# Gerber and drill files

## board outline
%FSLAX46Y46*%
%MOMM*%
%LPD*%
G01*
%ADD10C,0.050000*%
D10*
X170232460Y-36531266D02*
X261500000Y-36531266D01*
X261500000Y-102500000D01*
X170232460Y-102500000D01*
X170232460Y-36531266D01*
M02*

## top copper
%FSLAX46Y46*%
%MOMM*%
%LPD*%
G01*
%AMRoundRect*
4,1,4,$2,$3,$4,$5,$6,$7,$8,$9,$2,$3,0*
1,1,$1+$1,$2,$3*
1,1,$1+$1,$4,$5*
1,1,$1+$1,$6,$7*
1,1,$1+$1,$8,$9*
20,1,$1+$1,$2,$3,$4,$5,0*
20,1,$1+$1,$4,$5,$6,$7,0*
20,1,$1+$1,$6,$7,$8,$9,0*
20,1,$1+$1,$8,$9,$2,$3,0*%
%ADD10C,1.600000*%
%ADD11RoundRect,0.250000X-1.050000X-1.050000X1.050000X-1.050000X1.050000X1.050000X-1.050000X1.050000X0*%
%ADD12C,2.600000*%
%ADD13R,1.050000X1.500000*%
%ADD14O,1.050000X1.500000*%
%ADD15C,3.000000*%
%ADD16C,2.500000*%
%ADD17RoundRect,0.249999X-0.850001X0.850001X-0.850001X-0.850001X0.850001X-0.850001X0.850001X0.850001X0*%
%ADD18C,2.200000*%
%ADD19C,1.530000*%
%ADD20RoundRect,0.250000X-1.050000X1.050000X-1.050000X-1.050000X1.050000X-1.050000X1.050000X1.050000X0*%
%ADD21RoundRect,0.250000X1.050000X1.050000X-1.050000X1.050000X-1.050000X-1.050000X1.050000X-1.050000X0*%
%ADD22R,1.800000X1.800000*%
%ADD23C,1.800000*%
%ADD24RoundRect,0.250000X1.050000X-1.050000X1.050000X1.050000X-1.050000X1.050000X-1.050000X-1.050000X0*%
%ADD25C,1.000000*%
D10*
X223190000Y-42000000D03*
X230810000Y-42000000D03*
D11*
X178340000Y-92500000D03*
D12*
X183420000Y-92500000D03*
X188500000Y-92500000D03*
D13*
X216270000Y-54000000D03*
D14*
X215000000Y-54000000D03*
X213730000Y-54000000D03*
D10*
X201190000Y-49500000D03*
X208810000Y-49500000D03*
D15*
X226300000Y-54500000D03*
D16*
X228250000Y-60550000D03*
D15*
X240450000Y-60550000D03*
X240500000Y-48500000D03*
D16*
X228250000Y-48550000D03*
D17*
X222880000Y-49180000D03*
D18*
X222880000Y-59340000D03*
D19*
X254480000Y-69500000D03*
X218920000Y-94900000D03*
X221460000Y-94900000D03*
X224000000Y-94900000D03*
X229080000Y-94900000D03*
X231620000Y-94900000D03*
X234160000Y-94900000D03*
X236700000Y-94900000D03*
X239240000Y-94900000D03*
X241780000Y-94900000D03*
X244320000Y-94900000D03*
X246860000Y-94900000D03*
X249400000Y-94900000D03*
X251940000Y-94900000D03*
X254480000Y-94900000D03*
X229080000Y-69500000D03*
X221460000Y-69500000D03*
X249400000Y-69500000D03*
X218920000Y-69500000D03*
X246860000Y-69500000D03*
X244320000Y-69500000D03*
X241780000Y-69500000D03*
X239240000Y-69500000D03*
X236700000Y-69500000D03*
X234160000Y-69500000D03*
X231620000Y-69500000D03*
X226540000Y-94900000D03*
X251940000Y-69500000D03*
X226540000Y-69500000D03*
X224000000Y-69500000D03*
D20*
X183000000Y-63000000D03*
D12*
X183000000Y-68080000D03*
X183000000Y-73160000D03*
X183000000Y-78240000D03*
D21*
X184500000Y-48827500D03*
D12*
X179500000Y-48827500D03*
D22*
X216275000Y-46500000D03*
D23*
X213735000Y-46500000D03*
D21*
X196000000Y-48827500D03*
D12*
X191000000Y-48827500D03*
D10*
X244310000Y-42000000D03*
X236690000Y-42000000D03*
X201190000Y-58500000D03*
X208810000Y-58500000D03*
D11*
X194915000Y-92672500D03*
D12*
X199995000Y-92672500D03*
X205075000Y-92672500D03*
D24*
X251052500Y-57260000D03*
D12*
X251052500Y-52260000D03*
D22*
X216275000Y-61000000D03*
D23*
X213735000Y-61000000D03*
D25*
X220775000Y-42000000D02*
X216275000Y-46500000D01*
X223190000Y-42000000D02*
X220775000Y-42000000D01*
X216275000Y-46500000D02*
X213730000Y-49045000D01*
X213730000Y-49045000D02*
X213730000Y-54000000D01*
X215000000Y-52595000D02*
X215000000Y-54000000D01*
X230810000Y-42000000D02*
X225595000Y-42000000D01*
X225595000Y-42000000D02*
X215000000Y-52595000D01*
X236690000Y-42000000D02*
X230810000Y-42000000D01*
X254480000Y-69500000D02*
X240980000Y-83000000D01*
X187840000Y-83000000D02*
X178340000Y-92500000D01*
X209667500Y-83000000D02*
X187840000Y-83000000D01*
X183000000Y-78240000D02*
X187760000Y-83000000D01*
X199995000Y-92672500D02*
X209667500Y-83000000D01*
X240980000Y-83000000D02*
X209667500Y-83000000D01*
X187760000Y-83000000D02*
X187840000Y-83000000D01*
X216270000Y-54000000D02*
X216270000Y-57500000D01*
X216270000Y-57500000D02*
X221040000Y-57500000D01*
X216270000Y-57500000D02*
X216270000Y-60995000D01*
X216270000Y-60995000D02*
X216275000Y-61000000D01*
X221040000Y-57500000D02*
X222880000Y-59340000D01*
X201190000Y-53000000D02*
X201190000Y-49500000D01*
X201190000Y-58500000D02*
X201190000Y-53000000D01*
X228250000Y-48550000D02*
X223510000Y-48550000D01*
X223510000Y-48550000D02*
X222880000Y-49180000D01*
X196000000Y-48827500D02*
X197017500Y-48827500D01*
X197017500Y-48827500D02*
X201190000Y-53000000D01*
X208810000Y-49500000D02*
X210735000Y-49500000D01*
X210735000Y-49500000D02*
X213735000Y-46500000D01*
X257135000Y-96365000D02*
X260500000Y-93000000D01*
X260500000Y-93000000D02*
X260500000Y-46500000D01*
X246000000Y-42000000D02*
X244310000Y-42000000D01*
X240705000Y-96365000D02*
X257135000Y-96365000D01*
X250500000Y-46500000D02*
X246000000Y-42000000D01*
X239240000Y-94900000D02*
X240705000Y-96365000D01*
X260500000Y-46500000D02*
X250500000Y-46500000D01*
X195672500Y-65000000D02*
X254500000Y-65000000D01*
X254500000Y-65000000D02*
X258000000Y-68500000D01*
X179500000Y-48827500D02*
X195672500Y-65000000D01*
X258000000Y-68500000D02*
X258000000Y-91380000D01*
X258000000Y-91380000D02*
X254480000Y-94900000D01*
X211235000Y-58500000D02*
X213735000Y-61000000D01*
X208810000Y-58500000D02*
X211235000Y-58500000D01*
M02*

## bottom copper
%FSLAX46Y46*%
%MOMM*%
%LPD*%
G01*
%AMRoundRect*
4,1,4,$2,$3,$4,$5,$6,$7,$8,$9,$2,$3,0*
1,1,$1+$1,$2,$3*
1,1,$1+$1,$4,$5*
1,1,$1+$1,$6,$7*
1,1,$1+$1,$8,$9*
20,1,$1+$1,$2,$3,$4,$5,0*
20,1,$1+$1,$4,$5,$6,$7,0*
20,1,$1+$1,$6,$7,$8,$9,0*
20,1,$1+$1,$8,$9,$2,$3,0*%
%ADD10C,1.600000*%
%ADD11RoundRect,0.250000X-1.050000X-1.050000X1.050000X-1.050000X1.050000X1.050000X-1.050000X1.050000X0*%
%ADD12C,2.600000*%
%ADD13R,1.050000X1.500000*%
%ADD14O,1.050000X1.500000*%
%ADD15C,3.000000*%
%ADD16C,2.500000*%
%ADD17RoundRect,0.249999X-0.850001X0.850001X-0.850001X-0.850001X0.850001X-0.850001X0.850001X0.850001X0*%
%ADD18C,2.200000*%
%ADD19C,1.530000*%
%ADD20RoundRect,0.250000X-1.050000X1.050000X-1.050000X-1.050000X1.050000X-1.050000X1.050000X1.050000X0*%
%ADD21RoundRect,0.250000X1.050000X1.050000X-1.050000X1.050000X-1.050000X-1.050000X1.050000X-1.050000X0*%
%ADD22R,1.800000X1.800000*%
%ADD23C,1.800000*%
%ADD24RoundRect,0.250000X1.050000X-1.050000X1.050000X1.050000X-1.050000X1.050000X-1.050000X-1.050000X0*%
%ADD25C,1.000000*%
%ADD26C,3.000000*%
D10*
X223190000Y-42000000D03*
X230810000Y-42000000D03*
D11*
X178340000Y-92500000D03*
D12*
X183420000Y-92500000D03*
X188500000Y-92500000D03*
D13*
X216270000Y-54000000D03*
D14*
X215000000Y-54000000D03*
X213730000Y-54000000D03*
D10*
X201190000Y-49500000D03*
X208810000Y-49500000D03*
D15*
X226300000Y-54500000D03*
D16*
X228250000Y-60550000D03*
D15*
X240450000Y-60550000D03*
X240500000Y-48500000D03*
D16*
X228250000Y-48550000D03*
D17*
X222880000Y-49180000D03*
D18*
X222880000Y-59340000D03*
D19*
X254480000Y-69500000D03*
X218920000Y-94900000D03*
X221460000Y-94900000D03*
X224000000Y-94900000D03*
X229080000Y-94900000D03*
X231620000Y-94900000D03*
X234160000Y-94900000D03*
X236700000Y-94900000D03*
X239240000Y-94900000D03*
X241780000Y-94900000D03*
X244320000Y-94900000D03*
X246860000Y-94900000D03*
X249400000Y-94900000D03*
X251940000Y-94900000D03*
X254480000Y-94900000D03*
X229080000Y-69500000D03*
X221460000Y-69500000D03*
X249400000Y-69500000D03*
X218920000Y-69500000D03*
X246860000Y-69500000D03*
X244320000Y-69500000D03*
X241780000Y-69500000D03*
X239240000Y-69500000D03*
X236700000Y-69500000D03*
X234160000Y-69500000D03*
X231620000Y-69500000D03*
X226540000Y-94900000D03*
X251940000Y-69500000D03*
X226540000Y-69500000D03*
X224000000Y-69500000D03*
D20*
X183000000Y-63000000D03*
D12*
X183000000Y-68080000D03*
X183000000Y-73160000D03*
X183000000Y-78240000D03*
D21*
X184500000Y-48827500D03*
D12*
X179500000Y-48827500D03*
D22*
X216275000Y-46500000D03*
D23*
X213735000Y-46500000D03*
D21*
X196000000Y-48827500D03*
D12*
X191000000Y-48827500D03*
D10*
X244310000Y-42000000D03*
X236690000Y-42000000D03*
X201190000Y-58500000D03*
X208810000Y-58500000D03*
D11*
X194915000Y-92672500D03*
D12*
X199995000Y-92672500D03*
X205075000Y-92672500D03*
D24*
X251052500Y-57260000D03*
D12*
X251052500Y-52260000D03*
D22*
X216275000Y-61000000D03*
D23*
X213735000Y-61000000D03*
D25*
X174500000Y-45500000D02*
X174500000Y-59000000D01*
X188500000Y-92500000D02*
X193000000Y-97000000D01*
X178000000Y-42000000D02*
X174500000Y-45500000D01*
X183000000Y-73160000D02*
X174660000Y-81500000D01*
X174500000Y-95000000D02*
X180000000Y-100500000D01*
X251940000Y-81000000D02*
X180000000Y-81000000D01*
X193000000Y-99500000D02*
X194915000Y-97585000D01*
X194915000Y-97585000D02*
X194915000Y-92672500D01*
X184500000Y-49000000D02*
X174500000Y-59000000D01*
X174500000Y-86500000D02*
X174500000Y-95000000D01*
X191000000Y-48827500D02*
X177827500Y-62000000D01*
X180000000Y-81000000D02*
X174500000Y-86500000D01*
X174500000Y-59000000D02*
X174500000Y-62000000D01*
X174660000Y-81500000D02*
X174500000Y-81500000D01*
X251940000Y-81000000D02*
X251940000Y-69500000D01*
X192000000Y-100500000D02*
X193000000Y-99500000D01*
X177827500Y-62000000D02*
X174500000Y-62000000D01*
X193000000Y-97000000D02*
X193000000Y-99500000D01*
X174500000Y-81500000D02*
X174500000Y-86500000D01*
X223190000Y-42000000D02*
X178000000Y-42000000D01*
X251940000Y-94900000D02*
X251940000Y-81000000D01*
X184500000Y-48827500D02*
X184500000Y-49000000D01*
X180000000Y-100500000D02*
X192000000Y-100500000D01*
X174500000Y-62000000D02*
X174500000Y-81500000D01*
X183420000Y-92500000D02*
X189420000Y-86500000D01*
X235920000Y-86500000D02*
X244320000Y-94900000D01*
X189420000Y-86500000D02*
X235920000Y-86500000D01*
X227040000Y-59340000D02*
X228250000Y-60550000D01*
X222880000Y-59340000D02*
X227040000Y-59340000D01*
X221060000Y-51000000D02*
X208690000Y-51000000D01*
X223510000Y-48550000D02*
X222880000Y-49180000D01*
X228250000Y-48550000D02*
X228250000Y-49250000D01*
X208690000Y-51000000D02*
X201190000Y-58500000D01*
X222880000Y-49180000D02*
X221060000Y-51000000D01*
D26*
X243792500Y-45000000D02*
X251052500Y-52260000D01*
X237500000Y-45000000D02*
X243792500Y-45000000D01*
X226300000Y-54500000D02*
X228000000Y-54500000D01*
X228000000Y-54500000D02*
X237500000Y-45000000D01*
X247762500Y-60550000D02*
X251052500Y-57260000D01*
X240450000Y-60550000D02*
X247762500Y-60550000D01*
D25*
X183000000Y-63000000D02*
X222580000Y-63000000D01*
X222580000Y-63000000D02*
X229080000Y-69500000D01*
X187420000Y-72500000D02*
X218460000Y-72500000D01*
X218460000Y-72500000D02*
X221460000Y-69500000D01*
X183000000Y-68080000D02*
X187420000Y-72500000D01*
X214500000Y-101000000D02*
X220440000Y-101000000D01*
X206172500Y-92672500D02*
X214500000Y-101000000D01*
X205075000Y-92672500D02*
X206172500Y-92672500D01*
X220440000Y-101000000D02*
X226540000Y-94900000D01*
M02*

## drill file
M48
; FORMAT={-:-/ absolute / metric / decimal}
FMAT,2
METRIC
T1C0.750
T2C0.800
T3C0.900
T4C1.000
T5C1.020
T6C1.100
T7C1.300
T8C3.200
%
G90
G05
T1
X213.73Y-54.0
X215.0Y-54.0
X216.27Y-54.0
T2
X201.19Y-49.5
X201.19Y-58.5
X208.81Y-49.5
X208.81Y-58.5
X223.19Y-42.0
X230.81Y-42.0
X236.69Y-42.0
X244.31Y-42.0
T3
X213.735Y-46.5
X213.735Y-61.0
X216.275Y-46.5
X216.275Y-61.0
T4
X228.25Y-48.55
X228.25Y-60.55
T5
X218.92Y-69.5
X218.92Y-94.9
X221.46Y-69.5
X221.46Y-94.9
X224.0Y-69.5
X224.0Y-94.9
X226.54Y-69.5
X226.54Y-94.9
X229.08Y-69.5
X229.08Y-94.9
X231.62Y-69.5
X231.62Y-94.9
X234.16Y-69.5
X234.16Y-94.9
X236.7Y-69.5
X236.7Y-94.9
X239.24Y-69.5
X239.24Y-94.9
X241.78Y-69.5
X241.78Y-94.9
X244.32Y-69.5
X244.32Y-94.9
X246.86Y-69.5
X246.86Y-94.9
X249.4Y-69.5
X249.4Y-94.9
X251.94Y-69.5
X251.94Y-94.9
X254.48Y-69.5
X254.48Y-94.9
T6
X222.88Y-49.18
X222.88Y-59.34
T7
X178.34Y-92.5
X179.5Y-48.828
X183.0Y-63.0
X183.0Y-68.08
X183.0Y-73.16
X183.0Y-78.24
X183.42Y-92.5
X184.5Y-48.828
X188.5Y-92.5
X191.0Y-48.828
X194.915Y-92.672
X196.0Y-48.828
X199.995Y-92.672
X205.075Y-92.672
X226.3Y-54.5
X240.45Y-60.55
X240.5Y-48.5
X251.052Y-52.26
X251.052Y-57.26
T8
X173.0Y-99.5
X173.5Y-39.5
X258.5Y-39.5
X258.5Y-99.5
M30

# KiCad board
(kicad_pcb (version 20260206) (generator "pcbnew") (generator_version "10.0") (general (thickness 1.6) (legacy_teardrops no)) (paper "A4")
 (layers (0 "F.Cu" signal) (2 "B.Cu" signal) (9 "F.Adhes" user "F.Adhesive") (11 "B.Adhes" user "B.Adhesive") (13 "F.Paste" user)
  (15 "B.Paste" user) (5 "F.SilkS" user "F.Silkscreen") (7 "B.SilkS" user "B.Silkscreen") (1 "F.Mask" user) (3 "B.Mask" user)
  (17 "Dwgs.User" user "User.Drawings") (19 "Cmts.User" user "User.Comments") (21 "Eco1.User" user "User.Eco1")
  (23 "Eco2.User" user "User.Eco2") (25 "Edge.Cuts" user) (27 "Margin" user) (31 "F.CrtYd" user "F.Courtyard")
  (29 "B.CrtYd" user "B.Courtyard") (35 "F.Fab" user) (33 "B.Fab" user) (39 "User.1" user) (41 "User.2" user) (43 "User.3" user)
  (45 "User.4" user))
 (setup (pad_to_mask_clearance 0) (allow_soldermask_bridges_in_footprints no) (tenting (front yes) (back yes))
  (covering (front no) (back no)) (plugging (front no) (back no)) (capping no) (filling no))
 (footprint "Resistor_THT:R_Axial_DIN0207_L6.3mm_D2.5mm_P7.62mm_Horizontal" (layer "F.Cu") (at 223.19 42)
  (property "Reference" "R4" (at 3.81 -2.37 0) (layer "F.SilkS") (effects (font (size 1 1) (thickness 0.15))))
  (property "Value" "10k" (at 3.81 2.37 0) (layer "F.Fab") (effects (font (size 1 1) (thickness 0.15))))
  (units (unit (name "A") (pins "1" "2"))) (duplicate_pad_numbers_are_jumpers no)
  (pad "1" thru_hole circle (at 0 0) (size 1.6 1.6) (drill 0.8) (layers "*.Cu" "*.Mask") (remove_unused_layers no) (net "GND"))
  (pad "2" thru_hole circle (at 7.62 0) (size 1.6 1.6) (drill 0.8) (layers "*.Cu" "*.Mask") (remove_unused_layers no) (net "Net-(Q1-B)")))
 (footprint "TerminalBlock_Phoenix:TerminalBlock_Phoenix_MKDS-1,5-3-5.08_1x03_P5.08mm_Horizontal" (layer "F.Cu") (at 178.34 92.5)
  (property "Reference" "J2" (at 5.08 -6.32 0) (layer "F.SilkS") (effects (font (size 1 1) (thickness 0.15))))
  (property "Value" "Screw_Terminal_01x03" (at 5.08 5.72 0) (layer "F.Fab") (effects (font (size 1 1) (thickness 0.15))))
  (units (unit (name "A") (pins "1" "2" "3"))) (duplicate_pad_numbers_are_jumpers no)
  (pad "1" thru_hole roundrect (at 0 0) (size 2.6 2.6) (drill 1.3) (layers "*.Cu" "*.Mask") (remove_unused_layers no)
   (roundrect_rratio 0.096154) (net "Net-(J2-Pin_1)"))
  (pad "2" thru_hole circle (at 5.08 0) (size 2.6 2.6) (drill 1.3) (layers "*.Cu" "*.Mask") (remove_unused_layers no) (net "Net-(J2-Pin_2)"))
  (pad "3" thru_hole circle (at 10.16 0) (size 2.6 2.6) (drill 1.3) (layers "*.Cu" "*.Mask") (remove_unused_layers no) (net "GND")))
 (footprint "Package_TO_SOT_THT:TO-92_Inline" (layer "F.Cu") (at 216.27 54 180)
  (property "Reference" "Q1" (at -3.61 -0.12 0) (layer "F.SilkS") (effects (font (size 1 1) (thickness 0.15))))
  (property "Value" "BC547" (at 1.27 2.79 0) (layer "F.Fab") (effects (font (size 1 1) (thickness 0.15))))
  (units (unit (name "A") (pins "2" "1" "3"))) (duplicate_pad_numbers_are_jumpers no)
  (pad "1" thru_hole rect (at 0 0 180) (size 1.05 1.5) (drill 0.75) (layers "*.Cu" "*.Mask") (remove_unused_layers no) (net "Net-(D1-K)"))
  (pad "2" thru_hole oval (at 1.27 0 180) (size 1.05 1.5) (drill 0.75) (layers "*.Cu" "*.Mask") (remove_unused_layers no) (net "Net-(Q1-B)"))
  (pad "3" thru_hole oval (at 2.54 0 180) (size 1.05 1.5) (drill 0.75) (layers "*.Cu" "*.Mask") (remove_unused_layers no) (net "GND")))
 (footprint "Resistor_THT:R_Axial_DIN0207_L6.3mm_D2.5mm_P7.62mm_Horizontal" (layer "F.Cu") (at 201.19 49.5)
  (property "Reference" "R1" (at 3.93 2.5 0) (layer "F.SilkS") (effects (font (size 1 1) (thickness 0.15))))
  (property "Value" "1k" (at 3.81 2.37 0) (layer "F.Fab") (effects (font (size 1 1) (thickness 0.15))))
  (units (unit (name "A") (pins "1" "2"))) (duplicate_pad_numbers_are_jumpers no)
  (pad "1" thru_hole circle (at 0 0) (size 1.6 1.6) (drill 0.8) (layers "*.Cu" "*.Mask") (remove_unused_layers no) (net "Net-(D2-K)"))
  (pad "2" thru_hole circle (at 7.62 0) (size 1.6 1.6) (drill 0.8) (layers "*.Cu" "*.Mask") (remove_unused_layers no) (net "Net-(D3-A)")))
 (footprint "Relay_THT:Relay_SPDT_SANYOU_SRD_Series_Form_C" (layer "F.Cu") (at 226.3 54.5)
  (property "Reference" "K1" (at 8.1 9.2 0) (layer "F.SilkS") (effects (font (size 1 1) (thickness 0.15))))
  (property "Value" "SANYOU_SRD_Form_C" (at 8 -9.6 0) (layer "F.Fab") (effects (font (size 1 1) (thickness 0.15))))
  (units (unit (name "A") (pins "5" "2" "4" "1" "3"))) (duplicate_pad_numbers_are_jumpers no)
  (pad "1" thru_hole circle (at 0 0 90) (size 3 3) (drill 1.3) (layers "*.Cu" "*.Mask") (remove_unused_layers no) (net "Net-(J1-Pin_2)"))
  (pad "2" thru_hole circle (at 1.95 6.05 90) (size 2.5 2.5) (drill 1) (layers "*.Cu" "*.Mask") (remove_unused_layers no) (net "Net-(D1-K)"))
  (pad "3" thru_hole circle (at 14.15 6.05 90) (size 3 3) (drill 1.3) (layers "*.Cu" "*.Mask") (remove_unused_layers no)
   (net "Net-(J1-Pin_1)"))
  (pad "4" thru_hole circle (at 14.2 -6 90) (size 3 3) (drill 1.3) (layers "*.Cu" "*.Mask") (remove_unused_layers no)
   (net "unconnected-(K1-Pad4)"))
  (pad "5" thru_hole circle (at 1.95 -5.95 90) (size 2.5 2.5) (drill 1) (layers "*.Cu" "*.Mask") (remove_unused_layers no)
   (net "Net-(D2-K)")))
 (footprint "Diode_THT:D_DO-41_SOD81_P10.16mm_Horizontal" (layer "F.Cu") (at 222.88 49.18 -90)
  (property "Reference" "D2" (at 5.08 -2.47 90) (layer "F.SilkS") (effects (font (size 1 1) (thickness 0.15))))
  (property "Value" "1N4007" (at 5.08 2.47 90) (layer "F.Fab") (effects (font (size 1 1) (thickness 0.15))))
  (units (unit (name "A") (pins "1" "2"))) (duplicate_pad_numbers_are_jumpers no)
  (pad "1" thru_hole roundrect (at 0 0 270) (size 2.2 2.2) (drill 1.1) (layers "*.Cu" "*.Mask") (remove_unused_layers no)
   (roundrect_rratio 0.113636) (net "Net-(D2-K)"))
  (pad "2" thru_hole circle (at 10.16 0 270) (size 2.2 2.2) (drill 1.1) (layers "*.Cu" "*.Mask") (remove_unused_layers no)
   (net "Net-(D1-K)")))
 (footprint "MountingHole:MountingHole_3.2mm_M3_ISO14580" (layer "F.Cu") (at 258.5 39.5)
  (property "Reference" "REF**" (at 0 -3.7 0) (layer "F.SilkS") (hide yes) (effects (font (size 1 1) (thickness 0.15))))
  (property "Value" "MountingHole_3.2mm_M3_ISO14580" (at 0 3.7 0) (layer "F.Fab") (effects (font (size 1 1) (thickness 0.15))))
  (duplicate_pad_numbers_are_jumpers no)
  (pad "" np_thru_hole circle (at 0 0) (size 3.2 3.2) (drill 3.2) (layers "*.Cu" "*.Mask")))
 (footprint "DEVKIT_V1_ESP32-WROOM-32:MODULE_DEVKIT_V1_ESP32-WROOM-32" (layer "F.Cu") (at 231.61 82.2 90)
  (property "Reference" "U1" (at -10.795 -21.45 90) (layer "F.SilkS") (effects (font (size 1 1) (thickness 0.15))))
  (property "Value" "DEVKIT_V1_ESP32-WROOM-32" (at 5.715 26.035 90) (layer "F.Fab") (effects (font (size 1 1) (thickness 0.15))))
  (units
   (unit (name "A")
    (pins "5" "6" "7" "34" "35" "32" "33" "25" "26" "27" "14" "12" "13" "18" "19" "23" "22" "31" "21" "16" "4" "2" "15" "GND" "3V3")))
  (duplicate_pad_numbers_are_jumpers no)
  (pad "3V3" thru_hole circle (at 12.7 22.87 90) (size 1.53 1.53) (drill 1.02) (layers "*.Cu" "*.Mask") (remove_unused_layers no)
   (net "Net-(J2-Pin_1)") (solder_mask_margin 0.102))
  (pad "5" thru_hole circle (at -12.7 -12.69 90) (size 1.53 1.53) (drill 1.02) (layers "*.Cu" "*.Mask") (remove_unused_layers no)
   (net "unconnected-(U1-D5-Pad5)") (solder_mask_margin 0.102))
  (pad "6" thru_hole circle (at -12.7 -10.15 90) (size 1.53 1.53) (drill 1.02) (layers "*.Cu" "*.Mask") (remove_unused_layers no)
   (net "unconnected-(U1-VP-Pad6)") (solder_mask_margin 0.102))
  (pad "7" thru_hole circle (at -12.7 -7.61 90) (size 1.53 1.53) (drill 1.02) (layers "*.Cu" "*.Mask") (remove_unused_layers no)
   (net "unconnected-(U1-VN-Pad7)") (solder_mask_margin 0.102))
  (pad "9" thru_hole circle (at -12.7 -2.53 90) (size 1.53 1.53) (drill 1.02) (layers "*.Cu" "*.Mask") (remove_unused_layers no)
   (solder_mask_margin 0.102))
  (pad "10" thru_hole circle (at -12.7 0.01 90) (size 1.53 1.53) (drill 1.02) (layers "*.Cu" "*.Mask") (remove_unused_layers no)
   (solder_mask_margin 0.102))
  (pad "11" thru_hole circle (at -12.7 2.55 90) (size 1.53 1.53) (drill 1.02) (layers "*.Cu" "*.Mask") (remove_unused_layers no)
   (solder_mask_margin 0.102))
  (pad "12" thru_hole circle (at -12.7 5.09 90) (size 1.53 1.53) (drill 1.02) (layers "*.Cu" "*.Mask") (remove_unused_layers no)
   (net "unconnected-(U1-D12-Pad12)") (solder_mask_margin 0.102))
  (pad "13" thru_hole circle (at -12.7 7.63 90) (size 1.53 1.53) (drill 1.02) (layers "*.Cu" "*.Mask") (remove_unused_layers no)
   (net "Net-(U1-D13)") (solder_mask_margin 0.102))
  (pad "14" thru_hole circle (at -12.7 10.17 90) (size 1.53 1.53) (drill 1.02) (layers "*.Cu" "*.Mask") (remove_unused_layers no)
   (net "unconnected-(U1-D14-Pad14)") (solder_mask_margin 0.102))
  (pad "15" thru_hole circle (at -12.7 12.71 90) (size 1.53 1.53) (drill 1.02) (layers "*.Cu" "*.Mask") (remove_unused_layers no)
   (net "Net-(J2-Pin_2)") (solder_mask_margin 0.102))
  (pad "16" thru_hole circle (at -12.7 15.25 90) (size 1.53 1.53) (drill 1.02) (layers "*.Cu" "*.Mask") (remove_unused_layers no)
   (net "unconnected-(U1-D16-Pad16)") (solder_mask_margin 0.102))
  (pad "17" thru_hole circle (at -12.7 17.79 90) (size 1.53 1.53) (drill 1.02) (layers "*.Cu" "*.Mask") (remove_unused_layers no)
   (solder_mask_margin 0.102))
  (pad "18" thru_hole circle (at -12.7 20.33 90) (size 1.53 1.53) (drill 1.02) (layers "*.Cu" "*.Mask") (remove_unused_layers no)
   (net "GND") (solder_mask_margin 0.102))
  (pad "19" thru_hole circle (at -12.7 22.87 90) (size 1.53 1.53) (drill 1.02) (layers "*.Cu" "*.Mask") (remove_unused_layers no)
   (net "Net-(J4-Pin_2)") (solder_mask_margin 0.102))
  (pad "21" thru_hole circle (at 12.7 -2.53 90) (size 1.53 1.53) (drill 1.02) (layers "*.Cu" "*.Mask") (remove_unused_layers no)
   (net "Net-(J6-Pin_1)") (solder_mask_margin 0.102))
  (pad "22" thru_hole circle (at 12.7 -10.15 90) (size 1.53 1.53) (drill 1.02) (layers "*.Cu" "*.Mask") (remove_unused_layers no)
   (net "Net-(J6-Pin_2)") (solder_mask_margin 0.102))
  (pad "22" thru_hole circle (at 12.7 17.79 90) (size 1.53 1.53) (drill 1.02) (layers "*.Cu" "*.Mask") (remove_unused_layers no)
   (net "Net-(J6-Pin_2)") (solder_mask_margin 0.102))
  (pad "23" thru_hole circle (at 12.7 -12.69 90) (size 1.53 1.53) (drill 1.02) (layers "*.Cu" "*.Mask") (remove_unused_layers no)
   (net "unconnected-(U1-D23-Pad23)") (solder_mask_margin 0.102))
  (pad "23" thru_hole circle (at 12.7 15.25 90) (size 1.53 1.53) (drill 1.02) (layers "*.Cu" "*.Mask") (remove_unused_layers no)
   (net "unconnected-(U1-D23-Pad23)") (solder_mask_margin 0.102))
  (pad "24" thru_hole circle (at 12.7 12.71 90) (size 1.53 1.53) (drill 1.02) (layers "*.Cu" "*.Mask") (remove_unused_layers no)
   (solder_mask_margin 0.102))
  (pad "25" thru_hole circle (at 12.7 10.17 90) (size 1.53 1.53) (drill 1.02) (layers "*.Cu" "*.Mask") (remove_unused_layers no)
   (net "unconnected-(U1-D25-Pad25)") (solder_mask_margin 0.102))
  (pad "26" thru_hole circle (at 12.7 7.63 90) (size 1.53 1.53) (drill 1.02) (layers "*.Cu" "*.Mask") (remove_unused_layers no)
   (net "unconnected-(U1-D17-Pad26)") (solder_mask_margin 0.102))
  (pad "27" thru_hole circle (at 12.7 5.09 90) (size 1.53 1.53) (drill 1.02) (layers "*.Cu" "*.Mask") (remove_unused_layers no)
   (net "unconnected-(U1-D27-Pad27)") (solder_mask_margin 0.102))
  (pad "28" thru_hole circle (at 12.7 2.55 90) (size 1.53 1.53) (drill 1.02) (layers "*.Cu" "*.Mask") (remove_unused_layers no)
   (solder_mask_margin 0.102))
  (pad "29" thru_hole circle (at 12.7 0.01 90) (size 1.53 1.53) (drill 1.02) (layers "*.Cu" "*.Mask") (remove_unused_layers no)
   (solder_mask_margin 0.102))
  (pad "34" thru_hole circle (at -12.7 -5.07 90) (size 1.53 1.53) (drill 1.02) (layers "*.Cu" "*.Mask") (remove_unused_layers no)
   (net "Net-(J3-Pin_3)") (solder_mask_margin 0.102))
  (pad "GND" thru_hole circle (at 12.7 20.33 90) (size 1.53 1.53) (drill 1.02) (layers "*.Cu" "*.Mask") (remove_unused_layers no)
   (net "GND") (solder_mask_margin 0.102))
  (pad "RX0" thru_hole circle (at 12.7 -5.07 90) (size 1.53 1.53) (drill 1.02) (layers "*.Cu" "*.Mask") (remove_unused_layers no)
   (solder_mask_margin 0.102))
  (pad "TX0" thru_hole circle (at 12.7 -7.61 90) (size 1.53 1.53) (drill 1.02) (layers "*.Cu" "*.Mask") (remove_unused_layers no)
   (solder_mask_margin 0.102)))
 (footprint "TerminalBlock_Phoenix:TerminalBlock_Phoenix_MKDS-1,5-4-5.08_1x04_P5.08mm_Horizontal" (layer "F.Cu") (at 183 63 -90)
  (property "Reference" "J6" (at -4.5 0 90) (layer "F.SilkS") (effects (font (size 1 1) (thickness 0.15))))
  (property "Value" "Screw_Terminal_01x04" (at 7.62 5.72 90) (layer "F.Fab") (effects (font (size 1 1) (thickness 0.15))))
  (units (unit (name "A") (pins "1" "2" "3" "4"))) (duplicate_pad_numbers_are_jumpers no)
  (pad "1" thru_hole roundrect (at 0 0 270) (size 2.6 2.6) (drill 1.3) (layers "*.Cu" "*.Mask") (remove_unused_layers no)
   (roundrect_rratio 0.096154) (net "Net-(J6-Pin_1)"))
  (pad "2" thru_hole circle (at 5.08 0 270) (size 2.6 2.6) (drill 1.3) (layers "*.Cu" "*.Mask") (remove_unused_layers no)
   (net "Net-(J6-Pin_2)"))
  (pad "3" thru_hole circle (at 10.16 0 270) (size 2.6 2.6) (drill 1.3) (layers "*.Cu" "*.Mask") (remove_unused_layers no) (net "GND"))
  (pad "4" thru_hole circle (at 15.24 0 270) (size 2.6 2.6) (drill 1.3) (layers "*.Cu" "*.Mask") (remove_unused_layers no)
   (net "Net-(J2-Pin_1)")))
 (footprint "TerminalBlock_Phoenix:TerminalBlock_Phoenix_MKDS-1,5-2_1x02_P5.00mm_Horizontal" (layer "F.Cu") (at 184.5 48.8275 180)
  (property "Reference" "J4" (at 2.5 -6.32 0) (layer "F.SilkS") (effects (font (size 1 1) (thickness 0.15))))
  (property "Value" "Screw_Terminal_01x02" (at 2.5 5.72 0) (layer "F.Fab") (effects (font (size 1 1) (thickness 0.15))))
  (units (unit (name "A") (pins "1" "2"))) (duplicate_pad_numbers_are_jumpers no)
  (pad "1" thru_hole roundrect (at 0 0 180) (size 2.6 2.6) (drill 1.3) (layers "*.Cu" "*.Mask") (remove_unused_layers no)
   (roundrect_rratio 0.096154) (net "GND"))
  (pad "2" thru_hole circle (at 5 0 180) (size 2.6 2.6) (drill 1.3) (layers "*.Cu" "*.Mask") (remove_unused_layers no)
   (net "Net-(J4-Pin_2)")))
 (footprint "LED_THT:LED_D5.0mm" (layer "F.Cu") (at 216.275 46.5 180)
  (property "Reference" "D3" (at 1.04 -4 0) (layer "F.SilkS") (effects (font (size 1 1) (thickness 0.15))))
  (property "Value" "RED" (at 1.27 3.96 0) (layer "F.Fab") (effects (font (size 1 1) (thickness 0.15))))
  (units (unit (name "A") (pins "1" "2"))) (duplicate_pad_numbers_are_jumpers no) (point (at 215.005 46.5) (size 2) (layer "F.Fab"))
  (pad "1" thru_hole rect (at 0 0 180) (size 1.8 1.8) (drill 0.9) (layers "*.Cu" "*.Mask") (remove_unused_layers no) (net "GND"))
  (pad "2" thru_hole circle (at 2.54 0 180) (size 1.8 1.8) (drill 0.9) (layers "*.Cu" "*.Mask") (remove_unused_layers no) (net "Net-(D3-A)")))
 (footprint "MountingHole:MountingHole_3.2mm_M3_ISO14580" (layer "F.Cu") (at 258.5 99.5)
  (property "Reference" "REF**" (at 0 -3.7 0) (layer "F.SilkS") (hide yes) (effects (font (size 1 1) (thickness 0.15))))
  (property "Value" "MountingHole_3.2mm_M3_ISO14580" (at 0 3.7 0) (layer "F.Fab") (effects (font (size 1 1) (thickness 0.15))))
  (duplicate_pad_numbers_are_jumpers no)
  (pad "" np_thru_hole circle (at 0 0) (size 3.2 3.2) (drill 3.2) (layers "*.Cu" "*.Mask")))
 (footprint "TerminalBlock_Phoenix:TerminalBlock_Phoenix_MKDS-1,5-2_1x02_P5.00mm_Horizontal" (layer "F.Cu") (at 196 48.8275 180)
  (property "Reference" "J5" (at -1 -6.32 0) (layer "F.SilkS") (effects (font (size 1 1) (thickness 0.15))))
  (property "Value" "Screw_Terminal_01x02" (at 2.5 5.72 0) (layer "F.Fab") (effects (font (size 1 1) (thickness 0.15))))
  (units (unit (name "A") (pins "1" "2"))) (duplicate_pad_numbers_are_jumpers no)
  (pad "1" thru_hole roundrect (at 0 0 180) (size 2.6 2.6) (drill 1.3) (layers "*.Cu" "*.Mask") (remove_unused_layers no)
   (roundrect_rratio 0.096154) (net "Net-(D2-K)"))
  (pad "2" thru_hole circle (at 5 0 180) (size 2.6 2.6) (drill 1.3) (layers "*.Cu" "*.Mask") (remove_unused_layers no) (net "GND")))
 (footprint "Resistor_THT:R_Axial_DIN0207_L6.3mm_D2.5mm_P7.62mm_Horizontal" (layer "F.Cu") (at 244.31 42 180)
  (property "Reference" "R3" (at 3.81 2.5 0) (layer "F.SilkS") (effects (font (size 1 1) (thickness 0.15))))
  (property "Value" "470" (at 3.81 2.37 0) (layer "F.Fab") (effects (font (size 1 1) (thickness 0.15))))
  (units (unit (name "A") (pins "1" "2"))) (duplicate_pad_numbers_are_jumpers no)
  (pad "1" thru_hole circle (at 0 0 180) (size 1.6 1.6) (drill 0.8) (layers "*.Cu" "*.Mask") (remove_unused_layers no) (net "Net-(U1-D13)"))
  (pad "2" thru_hole circle (at 7.62 0 180) (size 1.6 1.6) (drill 0.8) (layers "*.Cu" "*.Mask") (remove_unused_layers no) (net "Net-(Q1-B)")))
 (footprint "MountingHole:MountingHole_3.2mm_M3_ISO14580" (layer "F.Cu") (at 173.5 39.5)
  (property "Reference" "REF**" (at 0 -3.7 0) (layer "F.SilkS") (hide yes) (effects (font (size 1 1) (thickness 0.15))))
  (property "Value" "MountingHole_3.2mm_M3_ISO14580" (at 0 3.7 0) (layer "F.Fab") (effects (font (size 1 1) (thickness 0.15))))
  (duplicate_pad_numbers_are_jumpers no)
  (pad "" np_thru_hole circle (at 0 0) (size 3.2 3.2) (drill 3.2) (layers "*.Cu" "*.Mask")))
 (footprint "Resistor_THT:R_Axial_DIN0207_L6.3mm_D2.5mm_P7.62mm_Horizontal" (layer "F.Cu") (at 201.19 58.5)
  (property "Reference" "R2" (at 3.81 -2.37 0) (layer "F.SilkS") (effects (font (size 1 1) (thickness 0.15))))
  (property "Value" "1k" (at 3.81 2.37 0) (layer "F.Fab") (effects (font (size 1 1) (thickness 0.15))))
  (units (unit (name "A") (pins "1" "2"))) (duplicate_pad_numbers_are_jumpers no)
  (pad "1" thru_hole circle (at 0 0) (size 1.6 1.6) (drill 0.8) (layers "*.Cu" "*.Mask") (remove_unused_layers no) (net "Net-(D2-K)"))
  (pad "2" thru_hole circle (at 7.62 0) (size 1.6 1.6) (drill 0.8) (layers "*.Cu" "*.Mask") (remove_unused_layers no) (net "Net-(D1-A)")))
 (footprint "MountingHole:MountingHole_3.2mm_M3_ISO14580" (layer "F.Cu") (at 173 99.5)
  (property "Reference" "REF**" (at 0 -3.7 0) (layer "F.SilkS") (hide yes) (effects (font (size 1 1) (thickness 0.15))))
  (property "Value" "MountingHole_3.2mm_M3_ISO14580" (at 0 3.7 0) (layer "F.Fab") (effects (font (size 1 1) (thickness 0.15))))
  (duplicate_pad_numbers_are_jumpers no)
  (pad "" np_thru_hole circle (at 0 0) (size 3.2 3.2) (drill 3.2) (layers "*.Cu" "*.Mask")))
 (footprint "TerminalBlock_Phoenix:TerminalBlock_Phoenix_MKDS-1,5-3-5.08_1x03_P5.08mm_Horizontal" (layer "F.Cu") (at 194.915 92.6725)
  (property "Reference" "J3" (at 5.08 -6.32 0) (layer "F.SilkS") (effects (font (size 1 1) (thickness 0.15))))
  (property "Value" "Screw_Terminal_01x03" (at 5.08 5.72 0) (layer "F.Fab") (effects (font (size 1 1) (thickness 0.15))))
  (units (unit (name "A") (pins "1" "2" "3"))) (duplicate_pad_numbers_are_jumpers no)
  (pad "1" thru_hole roundrect (at 0 0) (size 2.6 2.6) (drill 1.3) (layers "*.Cu" "*.Mask") (remove_unused_layers no)
   (roundrect_rratio 0.096154) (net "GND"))
  (pad "2" thru_hole circle (at 5.08 0) (size 2.6 2.6) (drill 1.3) (layers "*.Cu" "*.Mask") (remove_unused_layers no) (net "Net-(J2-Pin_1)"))
  (pad "3" thru_hole circle (at 10.16 0) (size 2.6 2.6) (drill 1.3) (layers "*.Cu" "*.Mask") (remove_unused_layers no)
   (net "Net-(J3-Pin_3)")))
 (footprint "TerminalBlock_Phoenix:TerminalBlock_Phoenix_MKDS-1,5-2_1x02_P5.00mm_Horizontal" (layer "F.Cu") (at 251.0525 57.26 90)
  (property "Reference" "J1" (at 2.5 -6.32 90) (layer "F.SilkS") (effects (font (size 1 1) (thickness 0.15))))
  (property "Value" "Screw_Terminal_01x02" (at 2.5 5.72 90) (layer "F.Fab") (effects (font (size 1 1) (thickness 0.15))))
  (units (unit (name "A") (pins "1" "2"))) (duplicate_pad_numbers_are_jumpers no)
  (pad "1" thru_hole roundrect (at 0 0 90) (size 2.6 2.6) (drill 1.3) (layers "*.Cu" "*.Mask") (remove_unused_layers no)
   (roundrect_rratio 0.096154) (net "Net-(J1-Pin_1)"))
  (pad "2" thru_hole circle (at 5 0 90) (size 2.6 2.6) (drill 1.3) (layers "*.Cu" "*.Mask") (remove_unused_layers no) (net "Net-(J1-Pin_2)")))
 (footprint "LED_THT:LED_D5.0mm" (layer "F.Cu") (at 216.275 61 180)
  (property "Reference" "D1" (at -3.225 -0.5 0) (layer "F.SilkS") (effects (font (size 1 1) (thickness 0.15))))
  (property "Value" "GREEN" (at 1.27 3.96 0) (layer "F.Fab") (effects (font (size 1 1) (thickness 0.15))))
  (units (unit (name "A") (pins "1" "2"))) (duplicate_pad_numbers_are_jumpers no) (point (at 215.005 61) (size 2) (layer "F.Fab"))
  (pad "1" thru_hole rect (at 0 0 180) (size 1.8 1.8) (drill 0.9) (layers "*.Cu" "*.Mask") (remove_unused_layers no) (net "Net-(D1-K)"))
  (pad "2" thru_hole circle (at 2.54 0 180) (size 1.8 1.8) (drill 0.9) (layers "*.Cu" "*.Mask") (remove_unused_layers no) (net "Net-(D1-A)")))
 (gr_rect (start 170.23246 36.531266) (end 261.5 102.5) (stroke (width 0.05) (type default)) (fill no) (layer "Edge.Cuts"))
 (segment (start 220.775 42) (end 216.275 46.5) (width 1) (layer "F.Cu") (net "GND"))
 (segment (start 223.19 42) (end 220.775 42) (width 1) (layer "F.Cu") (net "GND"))
 (segment (start 216.275 46.5) (end 213.73 49.045) (width 1) (layer "F.Cu") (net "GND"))
 (segment (start 213.73 49.045) (end 213.73 54) (width 1) (layer "F.Cu") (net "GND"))
 (segment (start 174.5 45.5) (end 174.5 59) (width 1) (layer "B.Cu") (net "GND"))
 (segment (start 188.5 92.5) (end 193 97) (width 1) (layer "B.Cu") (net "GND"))
 (segment (start 178 42) (end 174.5 45.5) (width 1) (layer "B.Cu") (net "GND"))
 (segment (start 183 73.16) (end 174.66 81.5) (width 1) (layer "B.Cu") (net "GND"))
 (segment (start 174.5 95) (end 180 100.5) (width 1) (layer "B.Cu") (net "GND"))
 (segment (start 251.94 81) (end 180 81) (width 1) (layer "B.Cu") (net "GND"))
 (segment (start 193 99.5) (end 194.915 97.585) (width 1) (layer "B.Cu") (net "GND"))
 (segment (start 194.915 97.585) (end 194.915 92.6725) (width 1) (layer "B.Cu") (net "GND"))
 (segment (start 184.5 49) (end 174.5 59) (width 1) (layer "B.Cu") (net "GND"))
 (segment (start 174.5 86.5) (end 174.5 95) (width 1) (layer "B.Cu") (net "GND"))
 (segment (start 191 48.8275) (end 177.8275 62) (width 1) (layer "B.Cu") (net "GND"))
 (segment (start 180 81) (end 174.5 86.5) (width 1) (layer "B.Cu") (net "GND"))
 (segment (start 174.5 59) (end 174.5 62) (width 1) (layer "B.Cu") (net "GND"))
 (segment (start 174.66 81.5) (end 174.5 81.5) (width 1) (layer "B.Cu") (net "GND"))
 (segment (start 251.94 81) (end 251.94 69.5) (width 1) (layer "B.Cu") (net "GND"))
 (segment (start 192 100.5) (end 193 99.5) (width 1) (layer "B.Cu") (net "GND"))
 (segment (start 177.8275 62) (end 174.5 62) (width 1) (layer "B.Cu") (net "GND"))
 (segment (start 193 97) (end 193 99.5) (width 1) (layer "B.Cu") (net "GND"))
 (segment (start 174.5 81.5) (end 174.5 86.5) (width 1) (layer "B.Cu") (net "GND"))
 (segment (start 223.19 42) (end 178 42) (width 1) (layer "B.Cu") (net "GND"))
 (segment (start 251.94 94.9) (end 251.94 81) (width 1) (layer "B.Cu") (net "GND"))
 (segment (start 184.5 48.8275) (end 184.5 49) (width 1) (layer "B.Cu") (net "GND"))
 (segment (start 180 100.5) (end 192 100.5) (width 1) (layer "B.Cu") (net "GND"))
 (segment (start 174.5 62) (end 174.5 81.5) (width 1) (layer "B.Cu") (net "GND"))
 (segment (start 215 52.595) (end 215 54) (width 1) (layer "F.Cu") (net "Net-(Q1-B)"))
 (segment (start 230.81 42) (end 225.595 42) (width 1) (layer "F.Cu") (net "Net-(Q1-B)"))
 (segment (start 225.595 42) (end 215 52.595) (width 1) (layer "F.Cu") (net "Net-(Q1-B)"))
 (segment (start 236.69 42) (end 230.81 42) (width 1) (layer "F.Cu") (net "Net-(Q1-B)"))
 (segment (start 254.48 69.5) (end 240.98 83) (width 1) (layer "F.Cu") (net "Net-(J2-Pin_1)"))
 (segment (start 187.84 83) (end 178.34 92.5) (width 1) (layer "F.Cu") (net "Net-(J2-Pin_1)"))
 (segment (start 209.6675 83) (end 187.84 83) (width 1) (layer "F.Cu") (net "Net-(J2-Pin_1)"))
 (segment (start 183 78.24) (end 187.76 83) (width 1) (layer "F.Cu") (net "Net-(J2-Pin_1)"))
 (segment (start 199.995 92.6725) (end 209.6675 83) (width 1) (layer "F.Cu") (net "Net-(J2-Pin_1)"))
 (segment (start 240.98 83) (end 209.6675 83) (width 1) (layer "F.Cu") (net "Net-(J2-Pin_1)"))
 (segment (start 187.76 83) (end 187.84 83) (width 1) (layer "F.Cu") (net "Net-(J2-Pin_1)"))
 (segment (start 183.42 92.5) (end 189.42 86.5) (width 1) (layer "B.Cu") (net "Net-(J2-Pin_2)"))
 (segment (start 235.92 86.5) (end 244.32 94.9) (width 1) (layer "B.Cu") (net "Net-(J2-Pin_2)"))
 (segment (start 189.42 86.5) (end 235.92 86.5) (width 1) (layer "B.Cu") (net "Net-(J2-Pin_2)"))
 (segment (start 216.27 54) (end 216.27 57.5) (width 1) (layer "F.Cu") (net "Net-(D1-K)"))
 (segment (start 216.27 57.5) (end 221.04 57.5) (width 1) (layer "F.Cu") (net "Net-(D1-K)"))
 (segment (start 216.27 57.5) (end 216.27 60.995) (width 1) (layer "F.Cu") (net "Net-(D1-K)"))
 (segment (start 216.27 60.995) (end 216.275 61) (width 1) (layer "F.Cu") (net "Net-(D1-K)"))
 (segment (start 221.04 57.5) (end 222.88 59.34) (width 1) (layer "F.Cu") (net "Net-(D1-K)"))
 (segment (start 227.04 59.34) (end 228.25 60.55) (width 1) (layer "B.Cu") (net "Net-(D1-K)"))
 (segment (start 222.88 59.34) (end 227.04 59.34) (width 1) (layer "B.Cu") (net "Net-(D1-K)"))
 (segment (start 201.19 53) (end 201.19 49.5) (width 1) (layer "F.Cu") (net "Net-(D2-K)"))
 (segment (start 201.19 58.5) (end 201.19 53) (width 1) (layer "F.Cu") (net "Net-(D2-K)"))
 (segment (start 228.25 48.55) (end 223.51 48.55) (width 1) (layer "F.Cu") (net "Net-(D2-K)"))
 (segment (start 223.51 48.55) (end 222.88 49.18) (width 1) (layer "F.Cu") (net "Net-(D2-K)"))
 (segment (start 196 48.8275) (end 197.0175 48.8275) (width 1) (layer "F.Cu") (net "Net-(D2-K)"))
 (segment (start 197.0175 48.8275) (end 201.19 53) (width 1) (layer "F.Cu") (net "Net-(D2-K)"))
 (segment (start 221.06 51) (end 208.69 51) (width 1) (layer "B.Cu") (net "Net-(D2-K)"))
 (segment (start 223.51 48.55) (end 222.88 49.18) (width 1) (layer "B.Cu") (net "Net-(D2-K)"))
 (segment (start 228.25 48.55) (end 228.25 49.25) (width 1) (layer "B.Cu") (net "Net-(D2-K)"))
 (segment (start 208.69 51) (end 201.19 58.5) (width 1) (layer "B.Cu") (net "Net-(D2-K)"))
 (segment (start 222.88 49.18) (end 221.06 51) (width 1) (layer "B.Cu") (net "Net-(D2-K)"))
 (segment (start 208.81 49.5) (end 210.735 49.5) (width 1) (layer "F.Cu") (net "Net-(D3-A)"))
 (segment (start 210.735 49.5) (end 213.735 46.5) (width 1) (layer "F.Cu") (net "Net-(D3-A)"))
 (segment (start 243.7925 45) (end 251.0525 52.26) (width 3) (layer "B.Cu") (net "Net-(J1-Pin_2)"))
 (segment (start 237.5 45) (end 243.7925 45) (width 3) (layer "B.Cu") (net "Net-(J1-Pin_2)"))
 (segment (start 226.3 54.5) (end 228 54.5) (width 3) (layer "B.Cu") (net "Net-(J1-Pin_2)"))
 (segment (start 228 54.5) (end 237.5 45) (width 3) (layer "B.Cu") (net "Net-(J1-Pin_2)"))
 (segment (start 247.7625 60.55) (end 251.0525 57.26) (width 3) (layer "B.Cu") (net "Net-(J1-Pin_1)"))
 (segment (start 240.45 60.55) (end 247.7625 60.55) (width 3) (layer "B.Cu") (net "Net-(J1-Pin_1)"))
 (segment (start 257.135 96.365) (end 260.5 93) (width 1) (layer "F.Cu") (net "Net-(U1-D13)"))
 (segment (start 260.5 93) (end 260.5 46.5) (width 1) (layer "F.Cu") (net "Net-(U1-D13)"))
 (segment (start 246 42) (end 244.31 42) (width 1) (layer "F.Cu") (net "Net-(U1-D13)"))
 (segment (start 240.705 96.365) (end 257.135 96.365) (width 1) (layer "F.Cu") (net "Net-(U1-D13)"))
 (segment (start 250.5 46.5) (end 246 42) (width 1) (layer "F.Cu") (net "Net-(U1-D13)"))
 (segment (start 239.24 94.9) (end 240.705 96.365) (width 1) (layer "F.Cu") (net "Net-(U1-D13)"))
 (segment (start 260.5 46.5) (end 250.5 46.5) (width 1) (layer "F.Cu") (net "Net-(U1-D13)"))
 (segment (start 195.6725 65) (end 254.5 65) (width 1) (layer "F.Cu") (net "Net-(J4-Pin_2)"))
 (segment (start 254.5 65) (end 258 68.5) (width 1) (layer "F.Cu") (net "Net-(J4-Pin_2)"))
 (segment (start 179.5 48.8275) (end 195.6725 65) (width 1) (layer "F.Cu") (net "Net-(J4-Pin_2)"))
 (segment (start 258 68.5) (end 258 91.38) (width 1) (layer "F.Cu") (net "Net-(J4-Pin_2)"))
 (segment (start 258 91.38) (end 254.48 94.9) (width 1) (layer "F.Cu") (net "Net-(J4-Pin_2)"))
 (segment (start 183 63) (end 222.58 63) (width 1) (layer "B.Cu") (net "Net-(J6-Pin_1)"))
 (segment (start 222.58 63) (end 229.08 69.5) (width 1) (layer "B.Cu") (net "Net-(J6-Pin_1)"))
 (segment (start 187.42 72.5) (end 218.46 72.5) (width 1) (layer "B.Cu") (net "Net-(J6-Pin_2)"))
 (segment (start 218.46 72.5) (end 221.46 69.5) (width 1) (layer "B.Cu") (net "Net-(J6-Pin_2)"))
 (segment (start 183 68.08) (end 187.42 72.5) (width 1) (layer "B.Cu") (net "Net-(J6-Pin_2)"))
 (segment (start 214.5 101) (end 220.44 101) (width 1) (layer "B.Cu") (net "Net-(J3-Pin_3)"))
 (segment (start 206.1725 92.6725) (end 214.5 101) (width 1) (layer "B.Cu") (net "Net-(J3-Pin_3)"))
 (segment (start 205.075 92.6725) (end 206.1725 92.6725) (width 1) (layer "B.Cu") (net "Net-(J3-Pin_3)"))
 (segment (start 220.44 101) (end 226.54 94.9) (width 1) (layer "B.Cu") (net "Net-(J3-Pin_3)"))
 (segment (start 211.235 58.5) (end 213.735 61) (width 1) (layer "F.Cu") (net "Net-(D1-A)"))
 (segment (start 208.81 58.5) (end 211.235 58.5) (width 1) (layer "F.Cu") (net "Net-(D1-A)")))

